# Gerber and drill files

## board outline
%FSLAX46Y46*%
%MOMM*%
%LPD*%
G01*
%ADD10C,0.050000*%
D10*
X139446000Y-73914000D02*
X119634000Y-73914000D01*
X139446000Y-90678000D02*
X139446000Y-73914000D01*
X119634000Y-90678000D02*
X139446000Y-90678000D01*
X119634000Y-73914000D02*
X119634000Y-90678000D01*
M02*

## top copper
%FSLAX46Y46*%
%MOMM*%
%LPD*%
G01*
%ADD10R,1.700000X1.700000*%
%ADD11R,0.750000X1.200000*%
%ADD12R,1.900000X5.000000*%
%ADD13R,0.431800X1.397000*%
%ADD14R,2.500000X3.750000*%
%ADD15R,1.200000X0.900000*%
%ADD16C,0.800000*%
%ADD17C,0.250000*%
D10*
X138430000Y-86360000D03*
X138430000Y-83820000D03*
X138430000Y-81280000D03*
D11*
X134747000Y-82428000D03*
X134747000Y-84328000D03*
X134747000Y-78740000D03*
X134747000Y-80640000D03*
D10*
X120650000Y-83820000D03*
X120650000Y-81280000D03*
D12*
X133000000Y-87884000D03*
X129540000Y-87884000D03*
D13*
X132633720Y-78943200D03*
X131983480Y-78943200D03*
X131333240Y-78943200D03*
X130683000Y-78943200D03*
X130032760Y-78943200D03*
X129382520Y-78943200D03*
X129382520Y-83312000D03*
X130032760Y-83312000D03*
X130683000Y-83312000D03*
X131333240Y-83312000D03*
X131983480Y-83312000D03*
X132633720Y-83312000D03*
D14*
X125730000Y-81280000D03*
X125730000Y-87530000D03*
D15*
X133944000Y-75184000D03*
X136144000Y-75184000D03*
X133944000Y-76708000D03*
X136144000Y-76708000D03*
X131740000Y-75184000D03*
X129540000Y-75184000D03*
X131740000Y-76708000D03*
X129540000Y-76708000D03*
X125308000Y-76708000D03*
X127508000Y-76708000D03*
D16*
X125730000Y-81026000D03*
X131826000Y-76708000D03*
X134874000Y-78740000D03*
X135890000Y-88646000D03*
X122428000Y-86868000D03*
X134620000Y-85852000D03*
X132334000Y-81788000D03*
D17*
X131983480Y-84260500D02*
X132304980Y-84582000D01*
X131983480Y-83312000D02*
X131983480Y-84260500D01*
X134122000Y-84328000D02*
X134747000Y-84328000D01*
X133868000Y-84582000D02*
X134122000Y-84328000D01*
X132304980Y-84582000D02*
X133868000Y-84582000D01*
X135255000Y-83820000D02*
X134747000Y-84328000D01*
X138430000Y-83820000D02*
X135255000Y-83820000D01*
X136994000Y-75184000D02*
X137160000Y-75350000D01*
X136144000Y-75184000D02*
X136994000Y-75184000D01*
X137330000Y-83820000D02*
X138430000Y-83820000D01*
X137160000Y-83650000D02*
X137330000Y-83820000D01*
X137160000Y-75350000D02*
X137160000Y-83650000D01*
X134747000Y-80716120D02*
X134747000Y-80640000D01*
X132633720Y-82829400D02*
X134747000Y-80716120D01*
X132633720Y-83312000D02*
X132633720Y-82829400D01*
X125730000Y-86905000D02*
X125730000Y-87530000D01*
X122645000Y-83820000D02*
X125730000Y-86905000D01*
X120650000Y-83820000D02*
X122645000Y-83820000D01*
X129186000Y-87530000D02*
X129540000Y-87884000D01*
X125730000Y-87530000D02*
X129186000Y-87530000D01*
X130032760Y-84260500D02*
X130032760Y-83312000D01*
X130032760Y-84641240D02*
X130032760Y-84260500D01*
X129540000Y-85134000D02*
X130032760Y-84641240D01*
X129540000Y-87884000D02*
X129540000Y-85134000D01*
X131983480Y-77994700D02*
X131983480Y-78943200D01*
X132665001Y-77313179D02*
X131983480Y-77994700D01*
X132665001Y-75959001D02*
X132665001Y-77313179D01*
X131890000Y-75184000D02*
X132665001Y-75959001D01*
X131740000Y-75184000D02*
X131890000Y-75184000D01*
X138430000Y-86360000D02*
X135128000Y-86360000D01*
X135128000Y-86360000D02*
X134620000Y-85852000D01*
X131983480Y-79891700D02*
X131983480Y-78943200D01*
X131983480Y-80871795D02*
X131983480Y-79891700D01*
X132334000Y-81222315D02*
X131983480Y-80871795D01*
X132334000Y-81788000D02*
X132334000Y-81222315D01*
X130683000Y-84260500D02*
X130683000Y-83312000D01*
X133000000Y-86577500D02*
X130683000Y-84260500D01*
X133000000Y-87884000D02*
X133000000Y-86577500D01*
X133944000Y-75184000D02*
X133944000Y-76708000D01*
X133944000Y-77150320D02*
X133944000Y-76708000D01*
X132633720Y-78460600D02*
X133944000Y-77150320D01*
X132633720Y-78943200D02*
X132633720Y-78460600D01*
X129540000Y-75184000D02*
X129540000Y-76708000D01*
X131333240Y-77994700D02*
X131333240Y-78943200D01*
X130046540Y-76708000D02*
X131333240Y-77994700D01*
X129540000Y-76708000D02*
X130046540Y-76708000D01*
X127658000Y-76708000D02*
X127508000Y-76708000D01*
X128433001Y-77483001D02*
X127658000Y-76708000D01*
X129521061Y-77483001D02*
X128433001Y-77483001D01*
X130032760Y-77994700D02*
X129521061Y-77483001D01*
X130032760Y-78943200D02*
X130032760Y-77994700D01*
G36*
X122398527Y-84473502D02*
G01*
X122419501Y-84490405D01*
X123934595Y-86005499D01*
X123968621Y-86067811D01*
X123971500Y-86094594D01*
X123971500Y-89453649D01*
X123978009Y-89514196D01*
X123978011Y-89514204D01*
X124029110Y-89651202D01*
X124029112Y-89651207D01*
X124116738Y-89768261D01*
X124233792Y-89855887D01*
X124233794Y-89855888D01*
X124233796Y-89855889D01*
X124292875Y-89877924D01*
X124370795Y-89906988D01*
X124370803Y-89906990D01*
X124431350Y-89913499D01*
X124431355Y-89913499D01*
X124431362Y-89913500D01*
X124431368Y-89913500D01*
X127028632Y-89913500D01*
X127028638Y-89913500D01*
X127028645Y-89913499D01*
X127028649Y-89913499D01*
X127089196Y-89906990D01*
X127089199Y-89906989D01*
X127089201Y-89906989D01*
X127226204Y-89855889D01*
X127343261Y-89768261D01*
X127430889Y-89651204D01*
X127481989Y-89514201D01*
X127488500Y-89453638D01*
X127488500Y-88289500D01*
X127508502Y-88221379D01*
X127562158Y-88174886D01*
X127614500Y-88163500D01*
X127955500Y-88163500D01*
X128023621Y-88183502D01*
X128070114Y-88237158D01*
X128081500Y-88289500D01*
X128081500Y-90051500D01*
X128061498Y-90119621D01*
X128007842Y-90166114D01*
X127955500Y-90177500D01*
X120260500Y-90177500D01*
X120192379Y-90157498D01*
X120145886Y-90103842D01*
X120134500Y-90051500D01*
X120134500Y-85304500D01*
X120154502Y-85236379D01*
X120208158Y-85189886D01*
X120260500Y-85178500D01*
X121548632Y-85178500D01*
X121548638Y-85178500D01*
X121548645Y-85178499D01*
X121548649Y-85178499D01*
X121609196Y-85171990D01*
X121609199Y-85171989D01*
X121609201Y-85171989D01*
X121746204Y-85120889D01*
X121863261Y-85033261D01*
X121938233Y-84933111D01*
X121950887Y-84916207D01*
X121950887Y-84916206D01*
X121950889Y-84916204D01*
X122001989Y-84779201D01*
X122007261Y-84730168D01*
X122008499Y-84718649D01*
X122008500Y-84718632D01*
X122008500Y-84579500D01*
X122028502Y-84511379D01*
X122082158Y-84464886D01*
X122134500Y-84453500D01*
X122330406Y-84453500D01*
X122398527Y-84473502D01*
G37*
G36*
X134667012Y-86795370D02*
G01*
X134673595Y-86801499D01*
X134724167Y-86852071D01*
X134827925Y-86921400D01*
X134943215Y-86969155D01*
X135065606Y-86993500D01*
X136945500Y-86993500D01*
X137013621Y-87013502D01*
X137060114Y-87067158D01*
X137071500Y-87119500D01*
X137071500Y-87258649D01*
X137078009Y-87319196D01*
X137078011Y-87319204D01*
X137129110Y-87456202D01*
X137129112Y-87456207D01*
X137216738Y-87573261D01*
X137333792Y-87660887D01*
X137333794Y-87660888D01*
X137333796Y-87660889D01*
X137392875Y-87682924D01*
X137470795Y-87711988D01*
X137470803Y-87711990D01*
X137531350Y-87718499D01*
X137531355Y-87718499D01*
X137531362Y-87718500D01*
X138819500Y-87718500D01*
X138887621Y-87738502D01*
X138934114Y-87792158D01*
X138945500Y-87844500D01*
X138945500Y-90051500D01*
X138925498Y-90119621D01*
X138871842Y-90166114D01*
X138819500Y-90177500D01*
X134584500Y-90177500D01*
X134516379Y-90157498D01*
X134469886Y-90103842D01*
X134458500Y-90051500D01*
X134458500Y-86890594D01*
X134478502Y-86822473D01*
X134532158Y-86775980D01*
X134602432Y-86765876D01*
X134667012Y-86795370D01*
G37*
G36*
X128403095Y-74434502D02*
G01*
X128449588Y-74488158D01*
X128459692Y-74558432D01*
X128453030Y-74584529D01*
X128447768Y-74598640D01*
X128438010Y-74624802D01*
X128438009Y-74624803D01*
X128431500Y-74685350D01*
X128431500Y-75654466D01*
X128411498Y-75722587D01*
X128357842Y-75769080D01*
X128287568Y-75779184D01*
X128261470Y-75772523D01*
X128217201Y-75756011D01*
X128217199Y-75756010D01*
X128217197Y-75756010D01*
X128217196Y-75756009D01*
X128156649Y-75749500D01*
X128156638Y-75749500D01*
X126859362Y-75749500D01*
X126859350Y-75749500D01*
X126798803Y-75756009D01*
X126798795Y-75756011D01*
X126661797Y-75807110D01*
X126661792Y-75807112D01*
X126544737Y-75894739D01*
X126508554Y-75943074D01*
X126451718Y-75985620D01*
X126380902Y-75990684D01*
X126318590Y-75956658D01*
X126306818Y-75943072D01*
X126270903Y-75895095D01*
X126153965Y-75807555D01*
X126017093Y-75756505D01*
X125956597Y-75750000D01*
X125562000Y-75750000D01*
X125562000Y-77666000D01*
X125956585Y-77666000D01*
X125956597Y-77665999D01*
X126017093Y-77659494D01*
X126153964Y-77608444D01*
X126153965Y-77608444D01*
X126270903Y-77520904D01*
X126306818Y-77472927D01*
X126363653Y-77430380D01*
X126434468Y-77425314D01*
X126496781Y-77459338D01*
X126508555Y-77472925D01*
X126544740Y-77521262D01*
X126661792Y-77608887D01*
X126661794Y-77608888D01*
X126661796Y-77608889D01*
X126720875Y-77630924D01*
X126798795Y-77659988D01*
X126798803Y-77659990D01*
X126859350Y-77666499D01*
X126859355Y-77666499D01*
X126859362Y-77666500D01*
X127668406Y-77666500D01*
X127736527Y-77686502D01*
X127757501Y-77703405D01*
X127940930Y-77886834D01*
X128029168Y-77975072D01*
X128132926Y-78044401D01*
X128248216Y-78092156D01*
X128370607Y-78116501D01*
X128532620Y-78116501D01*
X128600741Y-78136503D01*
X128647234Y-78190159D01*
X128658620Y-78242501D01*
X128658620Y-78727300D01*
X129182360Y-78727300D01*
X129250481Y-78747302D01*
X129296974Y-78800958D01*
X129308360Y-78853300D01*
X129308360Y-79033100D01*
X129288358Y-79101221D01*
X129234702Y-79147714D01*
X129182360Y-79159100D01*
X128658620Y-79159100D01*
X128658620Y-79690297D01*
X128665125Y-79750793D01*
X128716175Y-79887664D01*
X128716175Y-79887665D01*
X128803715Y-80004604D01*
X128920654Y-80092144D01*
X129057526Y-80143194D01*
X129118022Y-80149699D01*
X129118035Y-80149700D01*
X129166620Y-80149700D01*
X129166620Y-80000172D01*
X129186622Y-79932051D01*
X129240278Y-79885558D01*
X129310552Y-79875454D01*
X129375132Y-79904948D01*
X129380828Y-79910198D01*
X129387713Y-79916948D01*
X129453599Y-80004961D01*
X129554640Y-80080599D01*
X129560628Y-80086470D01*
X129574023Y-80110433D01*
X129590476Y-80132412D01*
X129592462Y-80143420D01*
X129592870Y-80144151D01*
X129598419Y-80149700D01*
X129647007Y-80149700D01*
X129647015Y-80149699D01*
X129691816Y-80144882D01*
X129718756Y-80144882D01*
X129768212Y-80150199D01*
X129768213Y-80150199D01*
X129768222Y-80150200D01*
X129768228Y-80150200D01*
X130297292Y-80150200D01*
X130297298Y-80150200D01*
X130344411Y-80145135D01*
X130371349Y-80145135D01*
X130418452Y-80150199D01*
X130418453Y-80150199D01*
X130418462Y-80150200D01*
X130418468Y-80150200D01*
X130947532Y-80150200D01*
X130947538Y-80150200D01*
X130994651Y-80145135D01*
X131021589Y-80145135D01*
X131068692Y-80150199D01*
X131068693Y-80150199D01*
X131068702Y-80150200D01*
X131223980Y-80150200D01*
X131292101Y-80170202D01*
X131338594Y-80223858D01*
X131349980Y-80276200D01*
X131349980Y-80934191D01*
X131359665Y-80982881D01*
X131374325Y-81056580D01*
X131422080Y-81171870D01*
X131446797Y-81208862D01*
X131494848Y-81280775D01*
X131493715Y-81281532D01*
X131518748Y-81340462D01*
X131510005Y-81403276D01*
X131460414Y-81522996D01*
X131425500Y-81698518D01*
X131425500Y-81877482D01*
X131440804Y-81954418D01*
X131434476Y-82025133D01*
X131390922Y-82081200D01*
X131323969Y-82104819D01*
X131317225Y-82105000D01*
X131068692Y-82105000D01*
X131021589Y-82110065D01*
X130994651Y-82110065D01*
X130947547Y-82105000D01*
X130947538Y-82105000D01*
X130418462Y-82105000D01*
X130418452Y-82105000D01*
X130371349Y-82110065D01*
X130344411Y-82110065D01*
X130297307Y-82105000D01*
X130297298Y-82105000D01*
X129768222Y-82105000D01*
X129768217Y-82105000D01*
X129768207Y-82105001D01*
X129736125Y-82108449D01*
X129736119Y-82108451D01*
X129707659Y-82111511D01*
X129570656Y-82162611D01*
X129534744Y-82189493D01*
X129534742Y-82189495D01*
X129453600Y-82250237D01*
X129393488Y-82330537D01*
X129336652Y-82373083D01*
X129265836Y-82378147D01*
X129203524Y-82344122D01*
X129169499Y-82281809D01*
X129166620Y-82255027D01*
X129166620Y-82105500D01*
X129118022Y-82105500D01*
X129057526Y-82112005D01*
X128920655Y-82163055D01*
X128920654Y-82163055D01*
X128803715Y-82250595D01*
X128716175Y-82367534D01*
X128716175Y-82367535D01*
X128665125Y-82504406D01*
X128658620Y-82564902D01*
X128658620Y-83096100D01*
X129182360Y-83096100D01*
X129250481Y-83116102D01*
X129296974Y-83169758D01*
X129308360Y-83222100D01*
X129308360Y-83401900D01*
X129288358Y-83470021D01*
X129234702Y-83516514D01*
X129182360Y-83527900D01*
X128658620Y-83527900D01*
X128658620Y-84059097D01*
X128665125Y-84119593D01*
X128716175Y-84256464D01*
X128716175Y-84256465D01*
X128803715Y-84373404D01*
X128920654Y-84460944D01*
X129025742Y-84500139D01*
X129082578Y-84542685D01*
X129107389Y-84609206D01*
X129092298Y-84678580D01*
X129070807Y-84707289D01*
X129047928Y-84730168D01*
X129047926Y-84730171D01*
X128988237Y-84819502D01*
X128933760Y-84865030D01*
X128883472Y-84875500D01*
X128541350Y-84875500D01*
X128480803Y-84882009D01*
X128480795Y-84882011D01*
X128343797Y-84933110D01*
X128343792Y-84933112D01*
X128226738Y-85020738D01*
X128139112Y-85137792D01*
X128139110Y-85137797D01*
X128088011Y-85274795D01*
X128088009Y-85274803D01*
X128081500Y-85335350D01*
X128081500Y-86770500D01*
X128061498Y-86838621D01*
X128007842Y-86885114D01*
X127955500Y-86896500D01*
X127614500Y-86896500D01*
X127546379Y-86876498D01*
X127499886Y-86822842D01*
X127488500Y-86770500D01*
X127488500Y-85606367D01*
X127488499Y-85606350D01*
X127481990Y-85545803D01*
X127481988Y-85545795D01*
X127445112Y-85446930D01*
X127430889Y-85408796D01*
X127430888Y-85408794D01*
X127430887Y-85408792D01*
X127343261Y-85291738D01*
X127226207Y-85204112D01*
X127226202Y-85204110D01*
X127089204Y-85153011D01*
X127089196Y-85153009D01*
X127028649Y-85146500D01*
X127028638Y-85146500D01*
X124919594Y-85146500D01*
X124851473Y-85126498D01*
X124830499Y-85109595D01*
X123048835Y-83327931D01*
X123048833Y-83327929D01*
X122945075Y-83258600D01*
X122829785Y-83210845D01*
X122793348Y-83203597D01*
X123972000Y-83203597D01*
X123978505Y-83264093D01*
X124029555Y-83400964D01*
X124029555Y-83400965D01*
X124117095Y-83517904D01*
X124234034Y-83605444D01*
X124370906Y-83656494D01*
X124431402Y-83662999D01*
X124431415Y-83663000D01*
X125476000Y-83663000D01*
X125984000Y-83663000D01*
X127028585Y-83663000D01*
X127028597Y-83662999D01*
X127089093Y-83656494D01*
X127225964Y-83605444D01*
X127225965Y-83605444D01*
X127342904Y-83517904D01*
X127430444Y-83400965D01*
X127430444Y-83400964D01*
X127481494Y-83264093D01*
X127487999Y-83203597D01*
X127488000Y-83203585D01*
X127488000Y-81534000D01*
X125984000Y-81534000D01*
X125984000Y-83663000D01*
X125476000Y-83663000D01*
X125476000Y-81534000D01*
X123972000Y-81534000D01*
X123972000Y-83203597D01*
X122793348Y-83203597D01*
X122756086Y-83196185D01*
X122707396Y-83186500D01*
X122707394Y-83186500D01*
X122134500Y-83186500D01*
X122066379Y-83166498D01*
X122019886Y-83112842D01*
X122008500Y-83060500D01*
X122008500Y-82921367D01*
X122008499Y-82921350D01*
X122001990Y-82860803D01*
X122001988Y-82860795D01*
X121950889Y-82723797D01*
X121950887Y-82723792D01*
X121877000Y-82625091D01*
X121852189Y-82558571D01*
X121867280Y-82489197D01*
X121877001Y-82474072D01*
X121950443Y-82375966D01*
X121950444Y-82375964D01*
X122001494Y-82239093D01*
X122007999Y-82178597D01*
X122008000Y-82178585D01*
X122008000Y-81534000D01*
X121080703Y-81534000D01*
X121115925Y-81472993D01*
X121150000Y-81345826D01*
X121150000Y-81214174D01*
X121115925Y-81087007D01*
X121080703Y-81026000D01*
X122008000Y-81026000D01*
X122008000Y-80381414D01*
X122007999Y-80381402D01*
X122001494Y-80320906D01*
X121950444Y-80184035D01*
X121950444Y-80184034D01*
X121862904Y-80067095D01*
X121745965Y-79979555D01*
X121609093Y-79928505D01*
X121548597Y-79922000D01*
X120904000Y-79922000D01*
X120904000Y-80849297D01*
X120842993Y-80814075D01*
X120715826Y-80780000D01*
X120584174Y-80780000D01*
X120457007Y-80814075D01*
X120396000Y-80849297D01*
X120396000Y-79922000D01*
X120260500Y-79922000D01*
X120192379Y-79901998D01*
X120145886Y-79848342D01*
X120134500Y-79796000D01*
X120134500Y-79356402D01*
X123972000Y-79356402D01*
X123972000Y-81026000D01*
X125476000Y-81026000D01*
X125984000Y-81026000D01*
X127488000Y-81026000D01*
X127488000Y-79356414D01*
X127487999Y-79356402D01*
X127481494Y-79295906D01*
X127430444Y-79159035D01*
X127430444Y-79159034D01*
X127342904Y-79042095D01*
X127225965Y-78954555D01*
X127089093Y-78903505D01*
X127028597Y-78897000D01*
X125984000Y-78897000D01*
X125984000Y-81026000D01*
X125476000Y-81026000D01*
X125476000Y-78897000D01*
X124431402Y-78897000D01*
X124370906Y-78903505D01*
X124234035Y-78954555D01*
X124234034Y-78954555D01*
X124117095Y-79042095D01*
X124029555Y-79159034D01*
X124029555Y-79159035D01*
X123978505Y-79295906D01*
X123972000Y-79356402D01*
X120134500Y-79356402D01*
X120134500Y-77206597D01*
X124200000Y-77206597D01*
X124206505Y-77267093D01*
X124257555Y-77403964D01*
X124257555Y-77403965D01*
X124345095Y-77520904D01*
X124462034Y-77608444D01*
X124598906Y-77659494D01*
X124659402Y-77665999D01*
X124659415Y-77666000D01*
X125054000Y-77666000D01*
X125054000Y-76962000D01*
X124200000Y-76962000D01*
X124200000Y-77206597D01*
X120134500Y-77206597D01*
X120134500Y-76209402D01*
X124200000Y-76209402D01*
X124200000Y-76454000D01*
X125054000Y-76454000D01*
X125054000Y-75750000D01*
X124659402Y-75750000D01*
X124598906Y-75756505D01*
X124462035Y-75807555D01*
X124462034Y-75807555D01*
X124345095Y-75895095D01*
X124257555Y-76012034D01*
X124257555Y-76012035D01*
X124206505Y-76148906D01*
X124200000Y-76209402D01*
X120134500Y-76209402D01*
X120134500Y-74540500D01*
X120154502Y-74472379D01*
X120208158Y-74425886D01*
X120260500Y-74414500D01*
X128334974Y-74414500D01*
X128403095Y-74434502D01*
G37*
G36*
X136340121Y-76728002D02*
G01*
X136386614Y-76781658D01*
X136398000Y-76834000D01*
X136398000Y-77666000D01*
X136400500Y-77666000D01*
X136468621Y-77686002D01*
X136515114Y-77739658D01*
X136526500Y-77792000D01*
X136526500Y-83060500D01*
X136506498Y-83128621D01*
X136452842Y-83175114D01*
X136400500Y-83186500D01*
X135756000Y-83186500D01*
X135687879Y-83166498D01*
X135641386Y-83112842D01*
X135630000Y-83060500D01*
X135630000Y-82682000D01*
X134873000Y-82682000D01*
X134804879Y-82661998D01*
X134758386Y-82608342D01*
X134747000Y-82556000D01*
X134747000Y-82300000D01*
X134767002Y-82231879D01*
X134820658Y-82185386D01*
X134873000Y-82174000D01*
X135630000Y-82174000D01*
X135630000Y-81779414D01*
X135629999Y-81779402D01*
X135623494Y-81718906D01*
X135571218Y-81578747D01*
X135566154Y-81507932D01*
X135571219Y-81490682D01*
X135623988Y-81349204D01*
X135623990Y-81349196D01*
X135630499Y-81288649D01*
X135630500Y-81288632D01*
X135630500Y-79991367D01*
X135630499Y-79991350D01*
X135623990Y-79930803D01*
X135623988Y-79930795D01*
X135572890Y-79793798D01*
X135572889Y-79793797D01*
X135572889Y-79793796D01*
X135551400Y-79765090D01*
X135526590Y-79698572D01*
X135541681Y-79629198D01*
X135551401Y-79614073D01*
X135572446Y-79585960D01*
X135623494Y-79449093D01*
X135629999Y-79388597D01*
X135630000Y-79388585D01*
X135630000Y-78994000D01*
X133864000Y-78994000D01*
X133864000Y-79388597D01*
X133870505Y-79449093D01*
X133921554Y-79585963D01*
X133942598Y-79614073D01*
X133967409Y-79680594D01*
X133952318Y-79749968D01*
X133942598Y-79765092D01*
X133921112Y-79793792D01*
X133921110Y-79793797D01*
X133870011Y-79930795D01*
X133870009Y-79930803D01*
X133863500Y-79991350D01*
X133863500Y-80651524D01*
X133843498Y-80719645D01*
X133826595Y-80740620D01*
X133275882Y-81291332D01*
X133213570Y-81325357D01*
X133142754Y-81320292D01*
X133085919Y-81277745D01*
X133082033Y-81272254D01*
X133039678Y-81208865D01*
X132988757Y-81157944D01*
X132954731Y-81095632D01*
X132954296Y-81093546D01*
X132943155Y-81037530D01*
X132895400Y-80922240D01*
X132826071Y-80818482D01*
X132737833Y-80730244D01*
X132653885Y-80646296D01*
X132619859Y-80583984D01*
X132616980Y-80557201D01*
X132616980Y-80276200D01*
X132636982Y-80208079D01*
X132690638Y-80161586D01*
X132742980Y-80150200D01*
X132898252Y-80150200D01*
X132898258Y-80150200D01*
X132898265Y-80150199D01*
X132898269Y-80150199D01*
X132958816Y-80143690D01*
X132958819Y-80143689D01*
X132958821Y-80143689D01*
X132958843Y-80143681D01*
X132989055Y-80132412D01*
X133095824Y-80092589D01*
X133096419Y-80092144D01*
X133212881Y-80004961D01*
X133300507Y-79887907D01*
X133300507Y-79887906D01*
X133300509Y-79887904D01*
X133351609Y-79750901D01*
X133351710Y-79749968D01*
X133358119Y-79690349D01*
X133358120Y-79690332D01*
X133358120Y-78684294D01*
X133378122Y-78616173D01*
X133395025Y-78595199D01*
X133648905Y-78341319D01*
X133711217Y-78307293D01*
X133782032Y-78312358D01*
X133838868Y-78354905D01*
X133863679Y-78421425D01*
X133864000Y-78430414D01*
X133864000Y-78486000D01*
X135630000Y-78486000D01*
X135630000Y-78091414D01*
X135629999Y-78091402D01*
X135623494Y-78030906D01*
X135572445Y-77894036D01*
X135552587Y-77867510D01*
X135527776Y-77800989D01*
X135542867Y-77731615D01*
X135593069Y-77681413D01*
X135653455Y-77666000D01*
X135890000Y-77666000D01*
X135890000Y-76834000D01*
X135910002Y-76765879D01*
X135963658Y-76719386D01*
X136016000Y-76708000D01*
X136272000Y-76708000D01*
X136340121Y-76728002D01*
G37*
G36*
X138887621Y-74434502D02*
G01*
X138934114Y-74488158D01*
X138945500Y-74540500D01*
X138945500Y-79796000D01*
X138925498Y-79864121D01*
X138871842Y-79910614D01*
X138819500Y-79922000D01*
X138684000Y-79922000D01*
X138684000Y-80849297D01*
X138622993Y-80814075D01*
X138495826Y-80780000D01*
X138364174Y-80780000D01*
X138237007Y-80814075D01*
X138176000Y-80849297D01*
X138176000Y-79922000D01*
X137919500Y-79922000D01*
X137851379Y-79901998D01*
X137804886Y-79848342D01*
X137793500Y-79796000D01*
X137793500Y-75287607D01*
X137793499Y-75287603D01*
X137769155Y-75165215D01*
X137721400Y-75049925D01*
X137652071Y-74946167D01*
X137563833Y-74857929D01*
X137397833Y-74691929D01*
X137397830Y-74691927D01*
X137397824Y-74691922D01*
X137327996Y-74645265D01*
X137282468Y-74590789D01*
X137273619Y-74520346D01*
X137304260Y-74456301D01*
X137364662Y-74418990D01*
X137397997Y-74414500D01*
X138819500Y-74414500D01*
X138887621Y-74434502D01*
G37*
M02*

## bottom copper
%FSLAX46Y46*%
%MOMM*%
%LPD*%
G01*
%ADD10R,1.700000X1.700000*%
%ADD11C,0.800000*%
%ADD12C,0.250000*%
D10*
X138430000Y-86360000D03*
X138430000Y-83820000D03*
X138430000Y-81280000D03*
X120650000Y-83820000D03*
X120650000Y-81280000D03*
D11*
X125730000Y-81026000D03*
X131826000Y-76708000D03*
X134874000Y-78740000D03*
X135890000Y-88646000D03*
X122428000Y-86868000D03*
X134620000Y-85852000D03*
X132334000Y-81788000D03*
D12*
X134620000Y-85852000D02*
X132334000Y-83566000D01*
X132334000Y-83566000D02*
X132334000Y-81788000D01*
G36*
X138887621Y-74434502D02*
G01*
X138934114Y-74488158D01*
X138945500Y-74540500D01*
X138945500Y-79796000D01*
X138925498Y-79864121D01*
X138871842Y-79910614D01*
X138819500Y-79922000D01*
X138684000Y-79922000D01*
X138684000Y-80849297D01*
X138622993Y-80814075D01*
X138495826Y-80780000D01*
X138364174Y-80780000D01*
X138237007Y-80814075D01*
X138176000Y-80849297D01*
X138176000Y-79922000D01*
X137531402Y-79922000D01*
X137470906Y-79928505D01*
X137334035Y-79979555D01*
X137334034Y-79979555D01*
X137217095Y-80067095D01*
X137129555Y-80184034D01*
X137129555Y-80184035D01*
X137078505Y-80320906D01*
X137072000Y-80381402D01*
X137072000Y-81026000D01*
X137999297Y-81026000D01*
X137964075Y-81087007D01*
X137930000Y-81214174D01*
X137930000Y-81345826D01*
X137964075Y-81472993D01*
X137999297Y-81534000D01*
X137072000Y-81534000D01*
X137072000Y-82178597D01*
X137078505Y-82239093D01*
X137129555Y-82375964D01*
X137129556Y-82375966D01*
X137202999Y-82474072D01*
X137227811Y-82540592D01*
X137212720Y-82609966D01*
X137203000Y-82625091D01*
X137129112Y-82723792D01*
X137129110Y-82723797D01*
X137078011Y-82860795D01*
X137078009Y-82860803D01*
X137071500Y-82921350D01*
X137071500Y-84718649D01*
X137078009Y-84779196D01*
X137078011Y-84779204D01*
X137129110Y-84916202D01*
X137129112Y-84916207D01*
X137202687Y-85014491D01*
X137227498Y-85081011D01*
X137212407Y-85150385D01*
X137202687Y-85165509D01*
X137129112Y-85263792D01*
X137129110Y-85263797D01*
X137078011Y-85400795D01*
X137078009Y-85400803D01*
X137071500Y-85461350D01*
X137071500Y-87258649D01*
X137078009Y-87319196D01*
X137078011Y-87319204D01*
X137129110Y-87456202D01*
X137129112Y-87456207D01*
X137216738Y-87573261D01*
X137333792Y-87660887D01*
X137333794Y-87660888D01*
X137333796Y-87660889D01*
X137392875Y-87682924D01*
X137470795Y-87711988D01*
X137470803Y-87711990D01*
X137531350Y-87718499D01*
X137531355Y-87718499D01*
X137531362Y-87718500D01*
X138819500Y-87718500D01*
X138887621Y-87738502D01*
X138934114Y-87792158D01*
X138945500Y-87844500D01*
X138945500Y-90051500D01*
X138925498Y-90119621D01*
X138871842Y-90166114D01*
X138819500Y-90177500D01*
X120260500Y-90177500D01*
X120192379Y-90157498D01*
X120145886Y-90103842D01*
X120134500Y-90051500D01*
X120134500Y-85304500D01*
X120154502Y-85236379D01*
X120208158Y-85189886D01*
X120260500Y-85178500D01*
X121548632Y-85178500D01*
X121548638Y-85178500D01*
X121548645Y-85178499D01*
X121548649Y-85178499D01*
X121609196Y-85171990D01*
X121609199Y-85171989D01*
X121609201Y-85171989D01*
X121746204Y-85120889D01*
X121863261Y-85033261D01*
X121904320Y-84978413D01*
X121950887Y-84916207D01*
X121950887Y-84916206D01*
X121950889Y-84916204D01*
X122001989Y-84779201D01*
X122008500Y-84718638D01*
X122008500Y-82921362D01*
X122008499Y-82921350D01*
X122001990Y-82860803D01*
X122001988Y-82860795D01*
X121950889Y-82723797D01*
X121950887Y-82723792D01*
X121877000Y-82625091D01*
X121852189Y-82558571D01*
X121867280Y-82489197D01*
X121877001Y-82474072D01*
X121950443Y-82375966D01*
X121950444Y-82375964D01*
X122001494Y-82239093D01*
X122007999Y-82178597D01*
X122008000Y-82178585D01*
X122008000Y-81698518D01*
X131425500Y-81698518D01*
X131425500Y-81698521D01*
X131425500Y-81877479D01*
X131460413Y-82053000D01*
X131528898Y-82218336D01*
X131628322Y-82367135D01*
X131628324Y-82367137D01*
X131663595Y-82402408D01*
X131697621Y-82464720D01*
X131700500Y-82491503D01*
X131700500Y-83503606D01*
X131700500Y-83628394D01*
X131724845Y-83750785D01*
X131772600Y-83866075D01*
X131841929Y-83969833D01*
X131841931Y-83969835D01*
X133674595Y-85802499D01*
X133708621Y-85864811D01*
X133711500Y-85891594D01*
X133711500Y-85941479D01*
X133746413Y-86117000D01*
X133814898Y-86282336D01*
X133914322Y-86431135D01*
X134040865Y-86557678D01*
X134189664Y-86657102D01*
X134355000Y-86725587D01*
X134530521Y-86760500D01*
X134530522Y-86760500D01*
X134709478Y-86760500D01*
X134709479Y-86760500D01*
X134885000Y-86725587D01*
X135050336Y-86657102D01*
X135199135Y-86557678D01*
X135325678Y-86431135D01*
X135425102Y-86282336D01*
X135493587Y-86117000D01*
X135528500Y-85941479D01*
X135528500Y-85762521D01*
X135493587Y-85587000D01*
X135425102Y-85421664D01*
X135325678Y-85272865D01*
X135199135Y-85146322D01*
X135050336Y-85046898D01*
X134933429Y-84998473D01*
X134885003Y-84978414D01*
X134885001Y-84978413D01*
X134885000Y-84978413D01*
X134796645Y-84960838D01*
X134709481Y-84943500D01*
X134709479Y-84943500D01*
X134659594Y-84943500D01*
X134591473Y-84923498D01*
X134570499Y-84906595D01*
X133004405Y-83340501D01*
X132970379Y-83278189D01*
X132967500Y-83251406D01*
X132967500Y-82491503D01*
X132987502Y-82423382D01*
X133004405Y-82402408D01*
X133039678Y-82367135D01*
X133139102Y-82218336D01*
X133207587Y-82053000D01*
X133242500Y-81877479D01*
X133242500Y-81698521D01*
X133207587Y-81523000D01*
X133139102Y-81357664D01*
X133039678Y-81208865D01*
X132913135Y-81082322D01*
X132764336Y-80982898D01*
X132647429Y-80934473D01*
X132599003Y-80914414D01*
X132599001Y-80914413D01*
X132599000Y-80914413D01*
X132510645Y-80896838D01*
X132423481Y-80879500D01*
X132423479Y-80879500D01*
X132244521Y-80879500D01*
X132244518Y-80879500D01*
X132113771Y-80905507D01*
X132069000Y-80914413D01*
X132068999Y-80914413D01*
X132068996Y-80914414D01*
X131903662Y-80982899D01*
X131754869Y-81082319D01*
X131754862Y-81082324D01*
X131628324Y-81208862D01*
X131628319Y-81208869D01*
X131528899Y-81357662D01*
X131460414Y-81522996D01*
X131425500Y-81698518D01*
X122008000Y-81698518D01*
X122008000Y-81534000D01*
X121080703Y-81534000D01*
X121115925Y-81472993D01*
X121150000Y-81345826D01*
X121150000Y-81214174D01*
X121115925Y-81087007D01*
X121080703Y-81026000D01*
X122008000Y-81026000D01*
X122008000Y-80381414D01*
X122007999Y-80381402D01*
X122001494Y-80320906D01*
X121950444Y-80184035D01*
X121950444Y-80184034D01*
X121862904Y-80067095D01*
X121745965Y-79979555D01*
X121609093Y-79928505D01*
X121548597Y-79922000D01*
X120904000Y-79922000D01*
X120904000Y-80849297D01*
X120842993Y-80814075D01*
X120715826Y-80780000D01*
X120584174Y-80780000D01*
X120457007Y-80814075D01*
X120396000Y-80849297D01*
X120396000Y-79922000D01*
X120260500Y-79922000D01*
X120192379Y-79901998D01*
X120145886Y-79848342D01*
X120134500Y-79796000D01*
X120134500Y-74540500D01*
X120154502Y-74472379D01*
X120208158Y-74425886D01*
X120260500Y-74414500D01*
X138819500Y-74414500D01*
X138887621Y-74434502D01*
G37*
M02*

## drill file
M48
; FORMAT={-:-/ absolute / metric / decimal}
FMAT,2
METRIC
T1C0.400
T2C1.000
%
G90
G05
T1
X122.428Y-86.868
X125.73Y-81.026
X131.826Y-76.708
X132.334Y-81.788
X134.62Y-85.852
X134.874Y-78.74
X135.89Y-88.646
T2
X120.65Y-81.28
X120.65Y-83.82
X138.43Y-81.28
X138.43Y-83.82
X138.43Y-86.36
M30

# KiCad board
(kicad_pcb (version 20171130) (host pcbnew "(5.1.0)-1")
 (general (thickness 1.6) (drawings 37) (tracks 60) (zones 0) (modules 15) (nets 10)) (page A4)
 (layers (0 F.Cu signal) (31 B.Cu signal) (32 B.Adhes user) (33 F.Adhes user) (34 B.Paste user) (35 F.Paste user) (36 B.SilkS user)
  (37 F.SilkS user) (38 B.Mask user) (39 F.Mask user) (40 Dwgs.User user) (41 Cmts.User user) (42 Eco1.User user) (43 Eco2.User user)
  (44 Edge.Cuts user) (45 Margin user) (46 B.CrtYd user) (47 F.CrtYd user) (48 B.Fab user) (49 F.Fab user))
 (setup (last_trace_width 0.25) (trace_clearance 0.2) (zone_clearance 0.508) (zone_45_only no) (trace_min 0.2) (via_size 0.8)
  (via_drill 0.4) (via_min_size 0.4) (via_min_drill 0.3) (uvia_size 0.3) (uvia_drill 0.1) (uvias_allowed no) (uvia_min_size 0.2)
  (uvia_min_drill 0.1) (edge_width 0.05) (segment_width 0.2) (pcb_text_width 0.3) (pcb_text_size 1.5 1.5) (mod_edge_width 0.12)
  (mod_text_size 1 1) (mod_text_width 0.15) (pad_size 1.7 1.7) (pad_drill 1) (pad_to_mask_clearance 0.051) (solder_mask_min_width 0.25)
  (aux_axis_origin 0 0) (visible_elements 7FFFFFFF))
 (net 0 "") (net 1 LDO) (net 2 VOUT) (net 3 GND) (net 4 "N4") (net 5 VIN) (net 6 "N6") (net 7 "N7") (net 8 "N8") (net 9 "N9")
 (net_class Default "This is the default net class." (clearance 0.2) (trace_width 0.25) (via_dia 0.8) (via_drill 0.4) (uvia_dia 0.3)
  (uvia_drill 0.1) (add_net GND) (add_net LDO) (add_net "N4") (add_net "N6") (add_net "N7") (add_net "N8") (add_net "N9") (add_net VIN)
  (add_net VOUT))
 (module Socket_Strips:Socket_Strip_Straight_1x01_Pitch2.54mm (layer F.Cu) (at 138.43 86.36)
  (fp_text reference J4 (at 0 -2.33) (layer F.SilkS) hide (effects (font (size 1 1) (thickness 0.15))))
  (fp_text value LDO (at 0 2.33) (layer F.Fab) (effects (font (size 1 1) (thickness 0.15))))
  (pad 1 thru_hole rect (at 0 0) (size 1.7 1.7) (drill 1) (layers *.Cu *.Mask) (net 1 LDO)))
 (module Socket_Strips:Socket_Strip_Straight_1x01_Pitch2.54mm (layer F.Cu) (at 138.43 83.82)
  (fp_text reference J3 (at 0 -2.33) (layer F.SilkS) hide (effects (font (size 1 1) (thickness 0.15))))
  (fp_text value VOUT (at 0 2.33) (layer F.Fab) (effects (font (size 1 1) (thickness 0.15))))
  (pad 1 thru_hole rect (at 0 0) (size 1.7 1.7) (drill 1) (layers *.Cu *.Mask) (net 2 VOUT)))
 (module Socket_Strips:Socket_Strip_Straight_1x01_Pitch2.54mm (layer F.Cu) (at 138.43 81.28)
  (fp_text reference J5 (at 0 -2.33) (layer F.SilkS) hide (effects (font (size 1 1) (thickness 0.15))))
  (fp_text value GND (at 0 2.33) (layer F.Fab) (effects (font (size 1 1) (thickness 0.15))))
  (pad 1 thru_hole rect (at 0 0) (size 1.7 1.7) (drill 1) (layers *.Cu *.Mask) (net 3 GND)))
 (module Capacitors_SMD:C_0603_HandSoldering (layer F.Cu) (at 134.747 83.378 90)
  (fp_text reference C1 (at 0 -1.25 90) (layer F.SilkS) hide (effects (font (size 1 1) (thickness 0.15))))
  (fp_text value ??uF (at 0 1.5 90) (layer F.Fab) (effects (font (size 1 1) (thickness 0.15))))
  (pad 2 smd rect (at 0.95 0 90) (size 1.2 0.75) (layers F.Cu F.Paste F.Mask) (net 3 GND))
  (pad 1 smd rect (at -0.95 0 90) (size 1.2 0.75) (layers F.Cu F.Paste F.Mask) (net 2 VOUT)))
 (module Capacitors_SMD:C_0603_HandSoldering (layer F.Cu) (at 134.747 79.69 90)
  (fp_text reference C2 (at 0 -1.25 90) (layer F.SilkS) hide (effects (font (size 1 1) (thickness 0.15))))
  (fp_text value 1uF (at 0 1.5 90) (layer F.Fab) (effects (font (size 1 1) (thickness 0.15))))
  (pad 2 smd rect (at 0.95 0 90) (size 1.2 0.75) (layers F.Cu F.Paste F.Mask) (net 3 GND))
  (pad 1 smd rect (at -0.95 0 90) (size 1.2 0.75) (layers F.Cu F.Paste F.Mask) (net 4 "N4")))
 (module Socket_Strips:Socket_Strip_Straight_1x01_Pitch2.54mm (layer F.Cu) (at 120.65 83.82)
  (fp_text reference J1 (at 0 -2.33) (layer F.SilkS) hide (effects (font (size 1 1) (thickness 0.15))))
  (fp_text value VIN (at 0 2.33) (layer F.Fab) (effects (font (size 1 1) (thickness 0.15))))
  (pad 1 thru_hole rect (at 0 0) (size 1.7 1.7) (drill 1) (layers *.Cu *.Mask) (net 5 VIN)))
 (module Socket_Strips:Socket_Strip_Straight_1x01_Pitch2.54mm (layer F.Cu) (at 120.65 81.28)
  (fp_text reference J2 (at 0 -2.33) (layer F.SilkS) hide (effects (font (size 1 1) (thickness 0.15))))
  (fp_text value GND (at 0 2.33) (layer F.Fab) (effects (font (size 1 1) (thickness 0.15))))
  (pad 1 thru_hole rect (at 0 0) (size 1.7 1.7) (drill 1) (layers *.Cu *.Mask) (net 3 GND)))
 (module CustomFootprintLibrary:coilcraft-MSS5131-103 (layer F.Cu) (at 131.27 87.884 180)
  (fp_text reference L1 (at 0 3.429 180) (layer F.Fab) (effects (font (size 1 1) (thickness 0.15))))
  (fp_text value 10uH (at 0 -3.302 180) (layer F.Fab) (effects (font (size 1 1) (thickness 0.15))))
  (pad 1 smd rect (at -1.73 0 180) (size 1.9 5) (layers F.Cu F.Paste F.Mask) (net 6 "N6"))
  (pad 2 smd rect (at 1.73 0 180) (size 1.9 5) (layers F.Cu F.Paste F.Mask) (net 5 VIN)))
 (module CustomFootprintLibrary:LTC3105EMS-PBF (layer F.Cu) (at 131.00812 81.1276 270)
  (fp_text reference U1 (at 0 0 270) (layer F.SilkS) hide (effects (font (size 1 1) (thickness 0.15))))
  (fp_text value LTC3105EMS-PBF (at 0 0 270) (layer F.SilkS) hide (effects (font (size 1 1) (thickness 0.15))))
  (pad 1 smd rect (at -2.1844 -1.6256 270) (size 1.397 0.4318) (layers F.Cu F.Paste F.Mask) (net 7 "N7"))
  (pad 2 smd rect (at -2.1844 -0.97536 270) (size 1.397 0.4318) (layers F.Cu F.Paste F.Mask) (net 1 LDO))
  (pad 3 smd rect (at -2.1844 -0.32512 270) (size 1.397 0.4318) (layers F.Cu F.Paste F.Mask) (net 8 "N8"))
  (pad 4 smd rect (at -2.1844 0.32512 270) (size 1.397 0.4318) (layers F.Cu F.Paste F.Mask))
  (pad 5 smd rect (at -2.1844 0.97536 270) (size 1.397 0.4318) (layers F.Cu F.Paste F.Mask) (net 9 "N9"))
  (pad 6 smd rect (at -2.1844 1.6256 270) (size 1.397 0.4318) (layers F.Cu F.Paste F.Mask) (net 3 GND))
  (pad 7 smd rect (at 2.1844 1.6256 270) (size 1.397 0.4318) (layers F.Cu F.Paste F.Mask) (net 3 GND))
  (pad 8 smd rect (at 2.1844 0.97536 270) (size 1.397 0.4318) (layers F.Cu F.Paste F.Mask) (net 5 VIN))
  (pad 9 smd rect (at 2.1844 0.32512 270) (size 1.397 0.4318) (layers F.Cu F.Paste F.Mask) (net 6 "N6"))
  (pad 10 smd rect (at 2.1844 -0.32512 270) (size 1.397 0.4318) (layers F.Cu F.Paste F.Mask))
  (pad 11 smd rect (at 2.1844 -0.97536 270) (size 1.397 0.4318) (layers F.Cu F.Paste F.Mask) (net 2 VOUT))
  (pad 12 smd rect (at 2.1844 -1.6256 270) (size 1.397 0.4318) (layers F.Cu F.Paste F.Mask) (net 4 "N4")))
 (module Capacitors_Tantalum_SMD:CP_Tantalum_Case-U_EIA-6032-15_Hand (layer F.Cu) (at 125.73 84.405 90)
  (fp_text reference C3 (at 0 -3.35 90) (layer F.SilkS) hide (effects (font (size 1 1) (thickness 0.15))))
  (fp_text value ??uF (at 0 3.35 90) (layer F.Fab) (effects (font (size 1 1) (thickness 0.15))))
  (pad 2 smd rect (at 3.125 0 90) (size 3.75 2.5) (layers F.Cu F.Paste F.Mask) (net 3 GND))
  (pad 1 smd rect (at -3.125 0 90) (size 3.75 2.5) (layers F.Cu F.Paste F.Mask) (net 5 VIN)))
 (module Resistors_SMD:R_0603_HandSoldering (layer F.Cu) (at 135.044 75.184 180)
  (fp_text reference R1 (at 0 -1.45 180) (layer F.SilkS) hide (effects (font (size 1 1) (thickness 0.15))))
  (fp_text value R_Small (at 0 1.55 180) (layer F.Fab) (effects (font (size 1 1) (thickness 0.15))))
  (pad 2 smd rect (at 1.1 0 180) (size 1.2 0.9) (layers F.Cu F.Paste F.Mask) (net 7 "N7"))
  (pad 1 smd rect (at -1.1 0 180) (size 1.2 0.9) (layers F.Cu F.Paste F.Mask) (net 2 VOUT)))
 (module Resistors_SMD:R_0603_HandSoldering (layer F.Cu) (at 135.044 76.708)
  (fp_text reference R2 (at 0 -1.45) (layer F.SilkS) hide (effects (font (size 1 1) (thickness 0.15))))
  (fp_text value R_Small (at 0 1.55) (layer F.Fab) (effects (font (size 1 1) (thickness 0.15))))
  (pad 1 smd rect (at -1.1 0) (size 1.2 0.9) (layers F.Cu F.Paste F.Mask) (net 7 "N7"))
  (pad 2 smd rect (at 1.1 0) (size 1.2 0.9) (layers F.Cu F.Paste F.Mask) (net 3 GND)))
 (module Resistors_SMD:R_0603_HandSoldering (layer F.Cu) (at 130.64 75.184 180)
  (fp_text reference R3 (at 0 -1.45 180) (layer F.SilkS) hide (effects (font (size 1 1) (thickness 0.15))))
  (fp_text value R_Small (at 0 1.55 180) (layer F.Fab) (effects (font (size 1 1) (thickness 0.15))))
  (pad 1 smd rect (at -1.1 0 180) (size 1.2 0.9) (layers F.Cu F.Paste F.Mask) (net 1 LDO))
  (pad 2 smd rect (at 1.1 0 180) (size 1.2 0.9) (layers F.Cu F.Paste F.Mask) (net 8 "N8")))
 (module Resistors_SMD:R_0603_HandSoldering (layer F.Cu) (at 130.64 76.708)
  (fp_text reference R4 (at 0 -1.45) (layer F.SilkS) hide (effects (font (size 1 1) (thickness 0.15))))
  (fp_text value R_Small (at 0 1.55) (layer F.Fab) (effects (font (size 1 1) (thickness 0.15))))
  (pad 2 smd rect (at 1.1 0) (size 1.2 0.9) (layers F.Cu F.Paste F.Mask) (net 3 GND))
  (pad 1 smd rect (at -1.1 0) (size 1.2 0.9) (layers F.Cu F.Paste F.Mask) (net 8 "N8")))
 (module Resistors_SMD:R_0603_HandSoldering (layer F.Cu) (at 126.408 76.708 180)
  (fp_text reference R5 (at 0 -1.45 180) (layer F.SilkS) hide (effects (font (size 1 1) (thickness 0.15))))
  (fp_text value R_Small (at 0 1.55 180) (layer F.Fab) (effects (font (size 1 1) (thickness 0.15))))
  (pad 2 smd rect (at 1.1 0 180) (size 1.2 0.9) (layers F.Cu F.Paste F.Mask) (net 3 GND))
  (pad 1 smd rect (at -1.1 0 180) (size 1.2 0.9) (layers F.Cu F.Paste F.Mask) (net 9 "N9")))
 (gr_line (start 139.446 73.914) (end 119.634 73.914) (layer Edge.Cuts) (width 0.05))
 (gr_line (start 139.446 90.678) (end 139.446 73.914) (layer Edge.Cuts) (width 0.05))
 (gr_line (start 119.634 90.678) (end 139.446 90.678) (layer Edge.Cuts) (width 0.05))
 (gr_line (start 119.634 73.914) (end 119.634 90.678) (layer Edge.Cuts) (width 0.05))
 (via (at 125.73 81.026) (size 0.8) (drill 0.4) (layers F.Cu B.Cu) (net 3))
 (via (at 131.826 76.708) (size 0.8) (drill 0.4) (layers F.Cu B.Cu) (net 3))
 (via (at 134.874 78.74) (size 0.8) (drill 0.4) (layers F.Cu B.Cu) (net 3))
 (via (at 135.89 88.646) (size 0.8) (drill 0.4) (layers F.Cu B.Cu) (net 3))
 (via (at 122.428 86.868) (size 0.8) (drill 0.4) (layers F.Cu B.Cu) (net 3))
 (segment (start 131.98348 84.2605) (end 132.30498 84.582) (width 0.25) (layer F.Cu) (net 2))
 (segment (start 131.98348 83.312) (end 131.98348 84.2605) (width 0.25) (layer F.Cu) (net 2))
 (segment (start 134.122 84.328) (end 134.747 84.328) (width 0.25) (layer F.Cu) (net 2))
 (segment (start 133.868 84.582) (end 134.122 84.328) (width 0.25) (layer F.Cu) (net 2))
 (segment (start 132.30498 84.582) (end 133.868 84.582) (width 0.25) (layer F.Cu) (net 2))
 (segment (start 135.255 83.82) (end 134.747 84.328) (width 0.25) (layer F.Cu) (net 2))
 (segment (start 138.43 83.82) (end 135.255 83.82) (width 0.25) (layer F.Cu) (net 2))
 (segment (start 136.994 75.184) (end 137.16 75.35) (width 0.25) (layer F.Cu) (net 2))
 (segment (start 136.144 75.184) (end 136.994 75.184) (width 0.25) (layer F.Cu) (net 2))
 (segment (start 137.33 83.82) (end 138.43 83.82) (width 0.25) (layer F.Cu) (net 2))
 (segment (start 137.16 83.65) (end 137.33 83.82) (width 0.25) (layer F.Cu) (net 2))
 (segment (start 137.16 75.35) (end 137.16 83.65) (width 0.25) (layer F.Cu) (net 2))
 (segment (start 134.747 80.71612) (end 134.747 80.64) (width 0.25) (layer F.Cu) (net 4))
 (segment (start 132.63372 82.8294) (end 134.747 80.71612) (width 0.25) (layer F.Cu) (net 4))
 (segment (start 132.63372 83.312) (end 132.63372 82.8294) (width 0.25) (layer F.Cu) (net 4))
 (segment (start 125.73 86.905) (end 125.73 87.53) (width 0.25) (layer F.Cu) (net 5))
 (segment (start 122.645 83.82) (end 125.73 86.905) (width 0.25) (layer F.Cu) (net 5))
 (segment (start 120.65 83.82) (end 122.645 83.82) (width 0.25) (layer F.Cu) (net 5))
 (segment (start 129.186 87.53) (end 129.54 87.884) (width 0.25) (layer F.Cu) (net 5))
 (segment (start 125.73 87.53) (end 129.186 87.53) (width 0.25) (layer F.Cu) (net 5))
 (segment (start 130.03276 84.2605) (end 130.03276 83.312) (width 0.25) (layer F.Cu) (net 5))
 (segment (start 130.03276 84.64124) (end 130.03276 84.2605) (width 0.25) (layer F.Cu) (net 5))
 (segment (start 129.54 85.134) (end 130.03276 84.64124) (width 0.25) (layer F.Cu) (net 5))
 (segment (start 129.54 87.884) (end 129.54 85.134) (width 0.25) (layer F.Cu) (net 5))
 (segment (start 131.98348 77.9947) (end 131.98348 78.9432) (width 0.25) (layer F.Cu) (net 1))
 (segment (start 132.665001 77.313179) (end 131.98348 77.9947) (width 0.25) (layer F.Cu) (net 1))
 (segment (start 132.665001 75.959001) (end 132.665001 77.313179) (width 0.25) (layer F.Cu) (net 1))
 (segment (start 131.89 75.184) (end 132.665001 75.959001) (width 0.25) (layer F.Cu) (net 1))
 (segment (start 131.74 75.184) (end 131.89 75.184) (width 0.25) (layer F.Cu) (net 1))
 (via (at 134.62 85.852) (size 0.8) (drill 0.4) (layers F.Cu B.Cu) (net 1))
 (segment (start 138.43 86.36) (end 135.128 86.36) (width 0.25) (layer F.Cu) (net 1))
 (segment (start 135.128 86.36) (end 134.62 85.852) (width 0.25) (layer F.Cu) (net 1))
 (via (at 132.334 81.788) (size 0.8) (drill 0.4) (layers F.Cu B.Cu) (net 1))
 (segment (start 134.62 85.852) (end 132.334 83.566) (width 0.25) (layer B.Cu) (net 1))
 (segment (start 132.334 83.566) (end 132.334 81.788) (width 0.25) (layer B.Cu) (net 1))
 (segment (start 131.98348 79.8917) (end 131.98348 78.9432) (width 0.25) (layer F.Cu) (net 1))
 (segment (start 131.98348 80.871795) (end 131.98348 79.8917) (width 0.25) (layer F.Cu) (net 1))
 (segment (start 132.334 81.222315) (end 131.98348 80.871795) (width 0.25) (layer F.Cu) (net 1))
 (segment (start 132.334 81.788) (end 132.334 81.222315) (width 0.25) (layer F.Cu) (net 1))
 (segment (start 130.683 84.2605) (end 130.683 83.312) (width 0.25) (layer F.Cu) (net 6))
 (segment (start 133 86.5775) (end 130.683 84.2605) (width 0.25) (layer F.Cu) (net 6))
 (segment (start 133 87.884) (end 133 86.5775) (width 0.25) (layer F.Cu) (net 6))
 (segment (start 133.944 75.184) (end 133.944 76.708) (width 0.25) (layer F.Cu) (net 7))
 (segment (start 133.944 77.15032) (end 133.944 76.708) (width 0.25) (layer F.Cu) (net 7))
 (segment (start 132.63372 78.4606) (end 133.944 77.15032) (width 0.25) (layer F.Cu) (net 7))
 (segment (start 132.63372 78.9432) (end 132.63372 78.4606) (width 0.25) (layer F.Cu) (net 7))
 (segment (start 129.54 75.184) (end 129.54 76.708) (width 0.25) (layer F.Cu) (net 8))
 (segment (start 131.33324 77.9947) (end 131.33324 78.9432) (width 0.25) (layer F.Cu) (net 8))
 (segment (start 130.04654 76.708) (end 131.33324 77.9947) (width 0.25) (layer F.Cu) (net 8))
 (segment (start 129.54 76.708) (end 130.04654 76.708) (width 0.25) (layer F.Cu) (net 8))
 (segment (start 127.658 76.708) (end 127.508 76.708) (width 0.25) (layer F.Cu) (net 9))
 (segment (start 128.433001 77.483001) (end 127.658 76.708) (width 0.25) (layer F.Cu) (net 9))
 (segment (start 129.521061 77.483001) (end 128.433001 77.483001) (width 0.25) (layer F.Cu) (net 9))
 (segment (start 130.03276 77.9947) (end 129.521061 77.483001) (width 0.25) (layer F.Cu) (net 9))
 (segment (start 130.03276 78.9432) (end 130.03276 77.9947) (width 0.25) (layer F.Cu) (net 9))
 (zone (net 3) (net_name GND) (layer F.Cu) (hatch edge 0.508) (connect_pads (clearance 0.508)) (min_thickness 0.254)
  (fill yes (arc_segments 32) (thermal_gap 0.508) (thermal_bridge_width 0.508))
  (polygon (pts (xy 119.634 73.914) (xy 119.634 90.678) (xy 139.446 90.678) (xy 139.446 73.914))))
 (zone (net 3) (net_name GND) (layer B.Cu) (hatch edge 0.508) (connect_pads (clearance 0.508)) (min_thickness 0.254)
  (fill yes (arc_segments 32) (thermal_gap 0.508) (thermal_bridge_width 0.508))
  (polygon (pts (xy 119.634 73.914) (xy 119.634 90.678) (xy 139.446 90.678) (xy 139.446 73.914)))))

